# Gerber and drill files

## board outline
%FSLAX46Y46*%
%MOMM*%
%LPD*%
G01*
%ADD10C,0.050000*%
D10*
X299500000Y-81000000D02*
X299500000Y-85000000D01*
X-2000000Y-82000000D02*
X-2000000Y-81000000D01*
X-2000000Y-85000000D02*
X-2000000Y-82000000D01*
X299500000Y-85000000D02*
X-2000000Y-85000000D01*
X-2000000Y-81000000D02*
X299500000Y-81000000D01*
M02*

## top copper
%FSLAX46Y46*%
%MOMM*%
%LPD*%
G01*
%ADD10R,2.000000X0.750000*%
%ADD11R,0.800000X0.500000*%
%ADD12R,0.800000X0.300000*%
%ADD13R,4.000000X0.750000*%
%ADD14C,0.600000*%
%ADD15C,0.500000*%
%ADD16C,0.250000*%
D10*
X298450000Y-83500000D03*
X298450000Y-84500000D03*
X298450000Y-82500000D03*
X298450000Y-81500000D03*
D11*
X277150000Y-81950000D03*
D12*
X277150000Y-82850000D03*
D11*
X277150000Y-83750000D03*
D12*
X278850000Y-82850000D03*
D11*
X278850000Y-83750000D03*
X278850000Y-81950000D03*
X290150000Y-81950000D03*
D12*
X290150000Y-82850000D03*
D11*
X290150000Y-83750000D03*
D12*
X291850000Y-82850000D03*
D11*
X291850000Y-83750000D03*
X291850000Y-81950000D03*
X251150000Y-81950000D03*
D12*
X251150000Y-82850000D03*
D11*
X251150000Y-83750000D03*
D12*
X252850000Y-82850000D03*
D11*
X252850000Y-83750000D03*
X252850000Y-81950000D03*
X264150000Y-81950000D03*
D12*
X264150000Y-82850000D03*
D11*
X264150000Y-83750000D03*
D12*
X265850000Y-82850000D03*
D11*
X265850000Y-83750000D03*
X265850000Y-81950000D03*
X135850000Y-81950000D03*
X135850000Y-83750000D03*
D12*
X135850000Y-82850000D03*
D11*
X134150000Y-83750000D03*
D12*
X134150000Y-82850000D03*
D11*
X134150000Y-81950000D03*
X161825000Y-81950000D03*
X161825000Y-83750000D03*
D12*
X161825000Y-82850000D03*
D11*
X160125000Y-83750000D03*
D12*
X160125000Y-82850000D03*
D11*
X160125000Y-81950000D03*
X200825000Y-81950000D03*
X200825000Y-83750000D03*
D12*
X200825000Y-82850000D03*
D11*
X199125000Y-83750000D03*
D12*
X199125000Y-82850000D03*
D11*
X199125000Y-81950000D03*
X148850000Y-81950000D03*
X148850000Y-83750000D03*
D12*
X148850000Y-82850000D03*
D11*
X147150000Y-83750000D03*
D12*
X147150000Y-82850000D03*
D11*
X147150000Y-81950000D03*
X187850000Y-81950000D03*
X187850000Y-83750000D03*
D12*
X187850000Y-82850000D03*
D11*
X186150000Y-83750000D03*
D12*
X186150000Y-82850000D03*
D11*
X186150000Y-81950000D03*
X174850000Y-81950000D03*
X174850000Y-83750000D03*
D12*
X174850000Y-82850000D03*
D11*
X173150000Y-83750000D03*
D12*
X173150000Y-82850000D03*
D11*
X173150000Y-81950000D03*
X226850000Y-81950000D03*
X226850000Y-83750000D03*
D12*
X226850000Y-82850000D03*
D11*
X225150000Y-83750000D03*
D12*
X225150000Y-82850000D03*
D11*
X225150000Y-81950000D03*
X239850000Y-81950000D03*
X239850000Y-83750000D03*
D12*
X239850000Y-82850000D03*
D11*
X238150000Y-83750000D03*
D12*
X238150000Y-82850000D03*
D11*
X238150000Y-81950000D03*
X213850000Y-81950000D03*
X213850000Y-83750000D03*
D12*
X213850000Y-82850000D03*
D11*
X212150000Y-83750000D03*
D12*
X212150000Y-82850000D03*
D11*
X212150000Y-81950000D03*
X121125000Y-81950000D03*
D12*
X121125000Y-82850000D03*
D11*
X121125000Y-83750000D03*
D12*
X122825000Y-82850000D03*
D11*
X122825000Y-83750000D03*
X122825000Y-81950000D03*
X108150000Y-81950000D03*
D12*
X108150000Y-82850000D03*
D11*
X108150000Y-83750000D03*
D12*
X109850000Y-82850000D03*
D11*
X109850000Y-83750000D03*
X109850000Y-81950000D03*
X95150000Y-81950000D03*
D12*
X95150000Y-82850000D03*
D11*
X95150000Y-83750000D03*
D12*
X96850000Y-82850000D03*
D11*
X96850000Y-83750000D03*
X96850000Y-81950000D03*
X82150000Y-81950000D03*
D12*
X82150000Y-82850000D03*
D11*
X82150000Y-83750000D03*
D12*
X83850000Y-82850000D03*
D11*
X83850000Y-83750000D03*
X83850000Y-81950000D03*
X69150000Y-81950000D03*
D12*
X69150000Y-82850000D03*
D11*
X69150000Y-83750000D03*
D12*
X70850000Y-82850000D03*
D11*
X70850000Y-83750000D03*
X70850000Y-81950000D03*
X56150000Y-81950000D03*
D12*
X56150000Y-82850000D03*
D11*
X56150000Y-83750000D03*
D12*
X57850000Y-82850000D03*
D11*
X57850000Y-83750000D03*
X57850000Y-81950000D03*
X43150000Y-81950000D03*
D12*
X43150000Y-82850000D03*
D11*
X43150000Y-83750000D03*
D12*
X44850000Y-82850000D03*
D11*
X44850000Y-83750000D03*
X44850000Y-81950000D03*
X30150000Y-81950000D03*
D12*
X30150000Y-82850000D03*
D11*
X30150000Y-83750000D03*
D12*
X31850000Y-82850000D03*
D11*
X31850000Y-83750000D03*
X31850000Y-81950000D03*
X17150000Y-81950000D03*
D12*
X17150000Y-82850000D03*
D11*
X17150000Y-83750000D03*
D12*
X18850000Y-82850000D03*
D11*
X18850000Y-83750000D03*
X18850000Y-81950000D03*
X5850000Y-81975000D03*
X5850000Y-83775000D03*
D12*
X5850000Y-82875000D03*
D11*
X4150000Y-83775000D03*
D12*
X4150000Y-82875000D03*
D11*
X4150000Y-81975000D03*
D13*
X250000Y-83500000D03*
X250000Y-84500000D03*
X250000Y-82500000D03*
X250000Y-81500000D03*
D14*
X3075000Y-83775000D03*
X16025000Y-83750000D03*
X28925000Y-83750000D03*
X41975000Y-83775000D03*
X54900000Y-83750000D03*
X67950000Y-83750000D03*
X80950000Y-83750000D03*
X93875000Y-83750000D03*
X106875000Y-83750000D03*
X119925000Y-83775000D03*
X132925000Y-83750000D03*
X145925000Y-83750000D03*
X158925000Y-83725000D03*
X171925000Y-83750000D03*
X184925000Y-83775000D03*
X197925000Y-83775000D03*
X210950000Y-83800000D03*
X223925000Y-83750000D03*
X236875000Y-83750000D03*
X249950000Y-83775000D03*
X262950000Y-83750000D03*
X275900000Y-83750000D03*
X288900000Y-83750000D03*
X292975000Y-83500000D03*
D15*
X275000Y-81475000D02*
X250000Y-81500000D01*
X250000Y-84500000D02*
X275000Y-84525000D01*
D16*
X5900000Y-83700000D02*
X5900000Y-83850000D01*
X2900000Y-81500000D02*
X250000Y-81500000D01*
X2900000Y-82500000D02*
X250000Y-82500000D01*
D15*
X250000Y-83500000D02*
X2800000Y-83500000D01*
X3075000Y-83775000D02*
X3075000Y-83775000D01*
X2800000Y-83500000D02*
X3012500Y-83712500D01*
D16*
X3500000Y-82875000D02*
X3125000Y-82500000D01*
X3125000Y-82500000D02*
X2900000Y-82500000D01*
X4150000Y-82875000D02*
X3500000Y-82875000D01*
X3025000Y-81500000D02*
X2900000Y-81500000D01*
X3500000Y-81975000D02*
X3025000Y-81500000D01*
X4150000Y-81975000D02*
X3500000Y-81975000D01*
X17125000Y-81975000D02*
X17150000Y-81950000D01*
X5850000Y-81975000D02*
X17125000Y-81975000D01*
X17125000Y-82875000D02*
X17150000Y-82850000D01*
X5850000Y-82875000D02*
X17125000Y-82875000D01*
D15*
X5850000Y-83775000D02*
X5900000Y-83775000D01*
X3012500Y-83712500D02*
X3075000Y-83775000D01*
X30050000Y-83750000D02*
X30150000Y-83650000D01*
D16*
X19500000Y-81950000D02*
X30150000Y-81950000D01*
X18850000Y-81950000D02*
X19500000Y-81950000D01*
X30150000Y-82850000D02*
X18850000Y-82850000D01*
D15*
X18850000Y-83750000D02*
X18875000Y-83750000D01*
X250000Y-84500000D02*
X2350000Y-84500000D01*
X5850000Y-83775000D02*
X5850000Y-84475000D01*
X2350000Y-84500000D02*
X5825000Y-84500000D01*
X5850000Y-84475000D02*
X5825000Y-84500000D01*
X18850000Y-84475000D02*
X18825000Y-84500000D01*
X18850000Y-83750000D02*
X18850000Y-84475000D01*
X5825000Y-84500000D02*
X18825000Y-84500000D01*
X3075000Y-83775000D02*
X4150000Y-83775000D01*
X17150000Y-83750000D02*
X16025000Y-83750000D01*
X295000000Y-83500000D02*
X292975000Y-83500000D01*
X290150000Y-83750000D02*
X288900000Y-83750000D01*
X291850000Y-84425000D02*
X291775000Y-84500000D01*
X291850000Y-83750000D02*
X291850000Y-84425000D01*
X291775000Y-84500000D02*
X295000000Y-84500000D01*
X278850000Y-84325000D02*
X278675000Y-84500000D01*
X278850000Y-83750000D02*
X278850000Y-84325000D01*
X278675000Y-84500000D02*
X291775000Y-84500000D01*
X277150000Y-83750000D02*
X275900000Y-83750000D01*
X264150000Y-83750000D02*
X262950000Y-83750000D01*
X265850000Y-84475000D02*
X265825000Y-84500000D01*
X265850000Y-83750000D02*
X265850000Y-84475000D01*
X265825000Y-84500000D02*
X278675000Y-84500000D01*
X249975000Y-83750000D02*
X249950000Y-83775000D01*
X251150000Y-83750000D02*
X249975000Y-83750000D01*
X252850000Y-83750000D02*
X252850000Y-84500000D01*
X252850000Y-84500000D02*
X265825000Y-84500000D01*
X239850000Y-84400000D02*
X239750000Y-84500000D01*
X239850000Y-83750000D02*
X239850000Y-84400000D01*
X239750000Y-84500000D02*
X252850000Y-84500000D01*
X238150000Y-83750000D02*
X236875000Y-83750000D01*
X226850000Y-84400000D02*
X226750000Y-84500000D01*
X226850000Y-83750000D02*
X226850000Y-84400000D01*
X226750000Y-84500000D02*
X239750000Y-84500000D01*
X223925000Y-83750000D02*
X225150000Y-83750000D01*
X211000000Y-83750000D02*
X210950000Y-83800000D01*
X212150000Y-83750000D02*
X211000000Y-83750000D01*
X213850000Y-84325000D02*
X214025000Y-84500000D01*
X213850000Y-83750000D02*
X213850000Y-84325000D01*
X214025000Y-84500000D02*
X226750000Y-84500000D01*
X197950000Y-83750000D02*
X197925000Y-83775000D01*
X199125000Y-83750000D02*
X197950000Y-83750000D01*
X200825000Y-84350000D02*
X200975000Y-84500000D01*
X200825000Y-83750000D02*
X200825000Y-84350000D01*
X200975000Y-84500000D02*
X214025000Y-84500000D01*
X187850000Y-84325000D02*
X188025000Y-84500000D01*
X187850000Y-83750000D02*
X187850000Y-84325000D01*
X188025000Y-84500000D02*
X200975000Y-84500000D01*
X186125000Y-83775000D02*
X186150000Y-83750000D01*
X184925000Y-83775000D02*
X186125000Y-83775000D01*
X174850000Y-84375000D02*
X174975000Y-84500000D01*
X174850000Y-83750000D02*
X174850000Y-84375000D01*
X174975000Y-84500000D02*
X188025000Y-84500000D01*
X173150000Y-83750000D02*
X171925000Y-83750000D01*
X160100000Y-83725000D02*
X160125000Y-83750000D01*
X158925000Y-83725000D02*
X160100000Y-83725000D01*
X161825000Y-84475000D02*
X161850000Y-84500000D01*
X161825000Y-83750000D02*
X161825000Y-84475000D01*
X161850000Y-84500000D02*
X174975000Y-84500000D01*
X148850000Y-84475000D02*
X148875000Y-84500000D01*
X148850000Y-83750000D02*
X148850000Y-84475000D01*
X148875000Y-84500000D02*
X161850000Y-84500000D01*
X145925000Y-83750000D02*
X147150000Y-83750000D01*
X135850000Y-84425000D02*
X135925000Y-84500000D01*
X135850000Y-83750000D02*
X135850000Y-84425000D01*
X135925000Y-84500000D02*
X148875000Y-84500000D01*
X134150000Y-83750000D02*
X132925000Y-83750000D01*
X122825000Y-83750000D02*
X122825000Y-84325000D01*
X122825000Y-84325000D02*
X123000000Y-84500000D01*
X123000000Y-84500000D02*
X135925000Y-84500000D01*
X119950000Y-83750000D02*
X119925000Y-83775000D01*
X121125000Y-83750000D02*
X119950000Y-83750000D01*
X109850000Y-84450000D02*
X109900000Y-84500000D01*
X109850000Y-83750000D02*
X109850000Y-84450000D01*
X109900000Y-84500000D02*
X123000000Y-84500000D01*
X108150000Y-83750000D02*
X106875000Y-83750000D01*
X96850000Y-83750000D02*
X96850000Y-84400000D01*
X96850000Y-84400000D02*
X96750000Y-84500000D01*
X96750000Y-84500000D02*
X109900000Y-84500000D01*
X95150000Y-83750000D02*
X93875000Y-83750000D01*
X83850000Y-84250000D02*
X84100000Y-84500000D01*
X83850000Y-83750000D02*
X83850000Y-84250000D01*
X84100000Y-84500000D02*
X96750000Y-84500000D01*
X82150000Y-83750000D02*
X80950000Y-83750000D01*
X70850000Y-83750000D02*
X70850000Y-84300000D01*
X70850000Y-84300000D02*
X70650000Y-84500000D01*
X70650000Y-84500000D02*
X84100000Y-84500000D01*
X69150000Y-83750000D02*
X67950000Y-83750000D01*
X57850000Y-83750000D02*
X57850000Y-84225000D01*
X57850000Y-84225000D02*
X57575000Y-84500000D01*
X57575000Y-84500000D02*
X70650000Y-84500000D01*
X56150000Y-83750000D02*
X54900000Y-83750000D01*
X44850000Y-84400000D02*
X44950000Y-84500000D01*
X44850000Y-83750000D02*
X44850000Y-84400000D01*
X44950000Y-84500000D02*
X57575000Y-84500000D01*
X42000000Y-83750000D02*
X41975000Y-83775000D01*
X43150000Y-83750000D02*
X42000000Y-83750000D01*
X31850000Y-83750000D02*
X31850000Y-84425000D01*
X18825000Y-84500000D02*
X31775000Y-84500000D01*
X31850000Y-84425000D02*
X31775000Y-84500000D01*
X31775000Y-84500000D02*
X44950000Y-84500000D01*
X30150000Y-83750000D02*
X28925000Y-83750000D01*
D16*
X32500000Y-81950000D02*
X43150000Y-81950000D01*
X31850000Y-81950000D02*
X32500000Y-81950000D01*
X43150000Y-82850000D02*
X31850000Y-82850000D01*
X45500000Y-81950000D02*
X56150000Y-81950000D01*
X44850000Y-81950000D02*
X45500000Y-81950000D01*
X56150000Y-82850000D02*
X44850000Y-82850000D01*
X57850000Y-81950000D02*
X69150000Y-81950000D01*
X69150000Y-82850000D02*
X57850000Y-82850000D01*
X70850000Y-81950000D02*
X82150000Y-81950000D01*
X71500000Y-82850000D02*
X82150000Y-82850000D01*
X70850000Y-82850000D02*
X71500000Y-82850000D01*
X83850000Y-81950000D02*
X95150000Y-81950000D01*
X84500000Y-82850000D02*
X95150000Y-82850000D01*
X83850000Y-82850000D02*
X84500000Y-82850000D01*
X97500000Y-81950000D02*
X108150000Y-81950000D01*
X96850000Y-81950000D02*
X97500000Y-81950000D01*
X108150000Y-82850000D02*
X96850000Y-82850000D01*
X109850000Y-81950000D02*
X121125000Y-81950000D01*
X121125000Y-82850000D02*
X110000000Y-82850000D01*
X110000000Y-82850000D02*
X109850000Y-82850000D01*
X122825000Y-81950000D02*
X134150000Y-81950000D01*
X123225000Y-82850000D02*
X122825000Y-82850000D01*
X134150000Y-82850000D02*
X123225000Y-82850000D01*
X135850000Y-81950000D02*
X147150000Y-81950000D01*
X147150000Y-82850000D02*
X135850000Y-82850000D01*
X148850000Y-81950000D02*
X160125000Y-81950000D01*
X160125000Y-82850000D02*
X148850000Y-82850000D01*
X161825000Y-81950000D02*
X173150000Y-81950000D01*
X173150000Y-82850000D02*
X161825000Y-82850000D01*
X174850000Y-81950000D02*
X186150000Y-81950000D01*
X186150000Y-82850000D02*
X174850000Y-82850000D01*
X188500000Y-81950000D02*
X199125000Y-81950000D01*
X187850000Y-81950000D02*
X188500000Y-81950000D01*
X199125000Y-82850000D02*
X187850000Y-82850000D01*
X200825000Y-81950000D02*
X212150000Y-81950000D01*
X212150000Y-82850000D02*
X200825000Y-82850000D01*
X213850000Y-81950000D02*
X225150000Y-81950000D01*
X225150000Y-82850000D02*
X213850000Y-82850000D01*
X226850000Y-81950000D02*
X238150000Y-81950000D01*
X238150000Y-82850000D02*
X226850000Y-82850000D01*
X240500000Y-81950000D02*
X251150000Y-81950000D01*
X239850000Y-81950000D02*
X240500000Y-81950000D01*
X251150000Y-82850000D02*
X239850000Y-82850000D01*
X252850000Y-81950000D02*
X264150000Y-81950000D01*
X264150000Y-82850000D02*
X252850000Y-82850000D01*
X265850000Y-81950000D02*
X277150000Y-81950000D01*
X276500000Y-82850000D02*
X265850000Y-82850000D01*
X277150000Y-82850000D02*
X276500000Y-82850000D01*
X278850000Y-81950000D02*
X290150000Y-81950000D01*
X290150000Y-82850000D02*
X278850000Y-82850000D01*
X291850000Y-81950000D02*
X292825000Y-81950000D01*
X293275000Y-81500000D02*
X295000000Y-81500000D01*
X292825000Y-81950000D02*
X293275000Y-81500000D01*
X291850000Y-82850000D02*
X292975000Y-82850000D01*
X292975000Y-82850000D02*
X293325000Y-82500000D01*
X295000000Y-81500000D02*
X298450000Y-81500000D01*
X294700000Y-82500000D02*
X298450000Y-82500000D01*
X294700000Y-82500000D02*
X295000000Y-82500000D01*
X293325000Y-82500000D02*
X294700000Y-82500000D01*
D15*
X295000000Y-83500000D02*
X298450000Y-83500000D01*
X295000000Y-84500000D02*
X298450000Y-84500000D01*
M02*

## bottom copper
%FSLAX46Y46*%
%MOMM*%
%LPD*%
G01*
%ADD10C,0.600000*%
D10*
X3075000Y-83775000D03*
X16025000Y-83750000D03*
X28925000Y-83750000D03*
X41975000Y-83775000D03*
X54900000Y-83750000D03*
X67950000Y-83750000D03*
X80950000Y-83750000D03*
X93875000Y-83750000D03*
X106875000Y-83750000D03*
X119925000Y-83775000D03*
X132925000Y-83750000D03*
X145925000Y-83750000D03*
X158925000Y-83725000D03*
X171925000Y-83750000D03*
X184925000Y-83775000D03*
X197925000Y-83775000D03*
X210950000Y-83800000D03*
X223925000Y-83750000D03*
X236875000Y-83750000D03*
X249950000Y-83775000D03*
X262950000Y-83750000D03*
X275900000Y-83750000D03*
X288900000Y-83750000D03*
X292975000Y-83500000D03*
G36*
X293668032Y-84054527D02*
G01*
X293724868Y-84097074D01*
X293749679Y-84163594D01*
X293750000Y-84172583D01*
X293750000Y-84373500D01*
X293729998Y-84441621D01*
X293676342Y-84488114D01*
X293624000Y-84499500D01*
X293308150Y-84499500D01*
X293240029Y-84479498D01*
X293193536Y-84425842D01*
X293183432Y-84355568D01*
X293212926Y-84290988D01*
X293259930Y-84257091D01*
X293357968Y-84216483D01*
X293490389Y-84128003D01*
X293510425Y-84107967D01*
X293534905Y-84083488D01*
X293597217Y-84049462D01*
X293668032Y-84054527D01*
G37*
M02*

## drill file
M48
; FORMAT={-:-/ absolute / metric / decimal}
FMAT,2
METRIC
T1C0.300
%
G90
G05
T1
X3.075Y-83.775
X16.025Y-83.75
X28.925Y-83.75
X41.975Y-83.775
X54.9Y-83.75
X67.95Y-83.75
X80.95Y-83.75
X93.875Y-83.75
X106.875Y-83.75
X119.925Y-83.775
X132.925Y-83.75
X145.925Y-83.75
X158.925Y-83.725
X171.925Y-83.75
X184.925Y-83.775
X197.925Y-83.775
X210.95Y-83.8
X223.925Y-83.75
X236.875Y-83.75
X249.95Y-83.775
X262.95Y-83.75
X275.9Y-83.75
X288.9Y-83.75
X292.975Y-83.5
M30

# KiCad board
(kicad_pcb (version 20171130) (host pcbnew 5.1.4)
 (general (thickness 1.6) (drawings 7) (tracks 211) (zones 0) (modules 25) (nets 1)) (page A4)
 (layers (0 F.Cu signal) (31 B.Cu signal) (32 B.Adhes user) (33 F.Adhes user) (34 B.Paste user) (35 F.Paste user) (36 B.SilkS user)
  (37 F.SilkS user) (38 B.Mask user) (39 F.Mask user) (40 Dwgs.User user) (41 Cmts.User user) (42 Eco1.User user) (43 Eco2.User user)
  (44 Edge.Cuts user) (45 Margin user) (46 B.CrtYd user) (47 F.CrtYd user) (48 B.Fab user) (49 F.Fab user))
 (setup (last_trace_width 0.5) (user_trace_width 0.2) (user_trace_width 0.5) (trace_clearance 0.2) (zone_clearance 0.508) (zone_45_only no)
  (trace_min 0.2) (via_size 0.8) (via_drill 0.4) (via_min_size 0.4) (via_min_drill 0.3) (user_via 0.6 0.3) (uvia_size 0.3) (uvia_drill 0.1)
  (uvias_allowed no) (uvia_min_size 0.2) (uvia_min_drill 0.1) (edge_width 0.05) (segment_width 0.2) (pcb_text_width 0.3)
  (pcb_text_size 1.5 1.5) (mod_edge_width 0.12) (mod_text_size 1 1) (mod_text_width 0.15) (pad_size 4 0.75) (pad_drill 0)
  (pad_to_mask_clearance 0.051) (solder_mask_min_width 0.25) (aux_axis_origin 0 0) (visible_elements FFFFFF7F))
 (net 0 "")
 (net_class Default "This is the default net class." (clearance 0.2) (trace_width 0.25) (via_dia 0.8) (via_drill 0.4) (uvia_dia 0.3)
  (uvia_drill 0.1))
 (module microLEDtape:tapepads (layer F.Cu) (at 281.2 81)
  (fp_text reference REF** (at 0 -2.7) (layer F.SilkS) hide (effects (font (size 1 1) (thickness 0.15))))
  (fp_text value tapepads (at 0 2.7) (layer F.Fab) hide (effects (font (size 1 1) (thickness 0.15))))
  (pad GND smd rect (at 17.25 2.5) (size 2 0.75) (layers F.Cu F.Paste F.Mask))
  (pad VCC smd rect (at 17.25 3.5) (size 2 0.75) (layers F.Cu F.Paste F.Mask))
  (pad CKI smd rect (at 17.25 1.5) (size 2 0.75) (layers F.Cu F.Paste F.Mask))
  (pad SDI smd rect (at 17.25 0.5) (size 2 0.75) (layers F.Cu F.Paste F.Mask)))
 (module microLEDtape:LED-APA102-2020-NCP (layer F.Cu) (at 278 82.85)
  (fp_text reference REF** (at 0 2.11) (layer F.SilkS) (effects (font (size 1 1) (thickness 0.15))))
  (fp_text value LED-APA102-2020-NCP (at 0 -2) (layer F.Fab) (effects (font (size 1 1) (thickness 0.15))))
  (pad SDI smd rect (at -0.85 -0.9) (size 0.8 0.5) (layers F.Cu F.Paste F.Mask))
  (pad CKI smd rect (at -0.85 0) (size 0.8 0.3) (layers F.Cu F.Paste F.Mask))
  (pad GND smd rect (at -0.85 0.9) (size 0.8 0.5) (layers F.Cu F.Paste F.Mask))
  (pad CKO smd rect (at 0.85 0) (size 0.8 0.3) (layers F.Cu F.Paste F.Mask))
  (pad VCC smd rect (at 0.85 0.9) (size 0.8 0.5) (layers F.Cu F.Paste F.Mask))
  (pad SDO smd rect (at 0.85 -0.9) (size 0.8 0.5) (layers F.Cu F.Paste F.Mask)))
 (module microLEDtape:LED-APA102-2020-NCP (layer F.Cu) (at 291 82.85)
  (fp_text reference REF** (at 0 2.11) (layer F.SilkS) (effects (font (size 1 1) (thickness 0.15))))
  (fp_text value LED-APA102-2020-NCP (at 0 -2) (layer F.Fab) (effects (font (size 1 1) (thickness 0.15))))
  (pad SDI smd rect (at -0.85 -0.9) (size 0.8 0.5) (layers F.Cu F.Paste F.Mask))
  (pad CKI smd rect (at -0.85 0) (size 0.8 0.3) (layers F.Cu F.Paste F.Mask))
  (pad GND smd rect (at -0.85 0.9) (size 0.8 0.5) (layers F.Cu F.Paste F.Mask))
  (pad CKO smd rect (at 0.85 0) (size 0.8 0.3) (layers F.Cu F.Paste F.Mask))
  (pad VCC smd rect (at 0.85 0.9) (size 0.8 0.5) (layers F.Cu F.Paste F.Mask))
  (pad SDO smd rect (at 0.85 -0.9) (size 0.8 0.5) (layers F.Cu F.Paste F.Mask)))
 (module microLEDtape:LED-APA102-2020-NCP (layer F.Cu) (at 252 82.85)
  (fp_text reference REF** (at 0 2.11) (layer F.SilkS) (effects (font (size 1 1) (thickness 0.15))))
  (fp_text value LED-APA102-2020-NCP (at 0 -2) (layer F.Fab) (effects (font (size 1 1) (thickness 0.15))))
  (pad SDI smd rect (at -0.85 -0.9) (size 0.8 0.5) (layers F.Cu F.Paste F.Mask))
  (pad CKI smd rect (at -0.85 0) (size 0.8 0.3) (layers F.Cu F.Paste F.Mask))
  (pad GND smd rect (at -0.85 0.9) (size 0.8 0.5) (layers F.Cu F.Paste F.Mask))
  (pad CKO smd rect (at 0.85 0) (size 0.8 0.3) (layers F.Cu F.Paste F.Mask))
  (pad VCC smd rect (at 0.85 0.9) (size 0.8 0.5) (layers F.Cu F.Paste F.Mask))
  (pad SDO smd rect (at 0.85 -0.9) (size 0.8 0.5) (layers F.Cu F.Paste F.Mask)))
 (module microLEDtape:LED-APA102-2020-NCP (layer F.Cu) (at 265 82.85)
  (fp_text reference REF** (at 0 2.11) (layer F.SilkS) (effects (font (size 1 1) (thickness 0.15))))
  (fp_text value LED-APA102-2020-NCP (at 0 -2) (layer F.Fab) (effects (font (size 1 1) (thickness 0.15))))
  (pad SDI smd rect (at -0.85 -0.9) (size 0.8 0.5) (layers F.Cu F.Paste F.Mask))
  (pad CKI smd rect (at -0.85 0) (size 0.8 0.3) (layers F.Cu F.Paste F.Mask))
  (pad GND smd rect (at -0.85 0.9) (size 0.8 0.5) (layers F.Cu F.Paste F.Mask))
  (pad CKO smd rect (at 0.85 0) (size 0.8 0.3) (layers F.Cu F.Paste F.Mask))
  (pad VCC smd rect (at 0.85 0.9) (size 0.8 0.5) (layers F.Cu F.Paste F.Mask))
  (pad SDO smd rect (at 0.85 -0.9) (size 0.8 0.5) (layers F.Cu F.Paste F.Mask)))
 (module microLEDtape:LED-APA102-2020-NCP (layer F.Cu) (at 135 82.85)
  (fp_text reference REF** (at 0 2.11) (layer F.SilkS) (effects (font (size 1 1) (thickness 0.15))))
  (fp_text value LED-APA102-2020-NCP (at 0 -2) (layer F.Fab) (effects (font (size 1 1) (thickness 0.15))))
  (pad SDO smd rect (at 0.85 -0.9) (size 0.8 0.5) (layers F.Cu F.Paste F.Mask))
  (pad VCC smd rect (at 0.85 0.9) (size 0.8 0.5) (layers F.Cu F.Paste F.Mask))
  (pad CKO smd rect (at 0.85 0) (size 0.8 0.3) (layers F.Cu F.Paste F.Mask))
  (pad GND smd rect (at -0.85 0.9) (size 0.8 0.5) (layers F.Cu F.Paste F.Mask))
  (pad CKI smd rect (at -0.85 0) (size 0.8 0.3) (layers F.Cu F.Paste F.Mask))
  (pad SDI smd rect (at -0.85 -0.9) (size 0.8 0.5) (layers F.Cu F.Paste F.Mask)))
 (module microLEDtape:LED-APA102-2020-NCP (layer F.Cu) (at 160.975 82.85)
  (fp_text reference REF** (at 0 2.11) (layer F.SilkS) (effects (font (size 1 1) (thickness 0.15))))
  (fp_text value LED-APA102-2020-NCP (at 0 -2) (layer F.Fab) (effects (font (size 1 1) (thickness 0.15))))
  (pad SDO smd rect (at 0.85 -0.9) (size 0.8 0.5) (layers F.Cu F.Paste F.Mask))
  (pad VCC smd rect (at 0.85 0.9) (size 0.8 0.5) (layers F.Cu F.Paste F.Mask))
  (pad CKO smd rect (at 0.85 0) (size 0.8 0.3) (layers F.Cu F.Paste F.Mask))
  (pad GND smd rect (at -0.85 0.9) (size 0.8 0.5) (layers F.Cu F.Paste F.Mask))
  (pad CKI smd rect (at -0.85 0) (size 0.8 0.3) (layers F.Cu F.Paste F.Mask))
  (pad SDI smd rect (at -0.85 -0.9) (size 0.8 0.5) (layers F.Cu F.Paste F.Mask)))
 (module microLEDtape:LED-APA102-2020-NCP (layer F.Cu) (at 199.975 82.85)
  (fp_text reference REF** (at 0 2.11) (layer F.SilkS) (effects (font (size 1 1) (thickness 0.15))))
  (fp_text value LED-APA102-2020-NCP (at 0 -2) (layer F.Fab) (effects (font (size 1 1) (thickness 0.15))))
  (pad SDO smd rect (at 0.85 -0.9) (size 0.8 0.5) (layers F.Cu F.Paste F.Mask))
  (pad VCC smd rect (at 0.85 0.9) (size 0.8 0.5) (layers F.Cu F.Paste F.Mask))
  (pad CKO smd rect (at 0.85 0) (size 0.8 0.3) (layers F.Cu F.Paste F.Mask))
  (pad GND smd rect (at -0.85 0.9) (size 0.8 0.5) (layers F.Cu F.Paste F.Mask))
  (pad CKI smd rect (at -0.85 0) (size 0.8 0.3) (layers F.Cu F.Paste F.Mask))
  (pad SDI smd rect (at -0.85 -0.9) (size 0.8 0.5) (layers F.Cu F.Paste F.Mask)))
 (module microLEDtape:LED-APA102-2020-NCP (layer F.Cu) (at 148 82.85)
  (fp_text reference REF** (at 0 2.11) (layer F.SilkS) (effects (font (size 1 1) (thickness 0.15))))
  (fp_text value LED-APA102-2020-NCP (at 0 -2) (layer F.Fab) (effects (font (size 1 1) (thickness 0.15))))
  (pad SDO smd rect (at 0.85 -0.9) (size 0.8 0.5) (layers F.Cu F.Paste F.Mask))
  (pad VCC smd rect (at 0.85 0.9) (size 0.8 0.5) (layers F.Cu F.Paste F.Mask))
  (pad CKO smd rect (at 0.85 0) (size 0.8 0.3) (layers F.Cu F.Paste F.Mask))
  (pad GND smd rect (at -0.85 0.9) (size 0.8 0.5) (layers F.Cu F.Paste F.Mask))
  (pad CKI smd rect (at -0.85 0) (size 0.8 0.3) (layers F.Cu F.Paste F.Mask))
  (pad SDI smd rect (at -0.85 -0.9) (size 0.8 0.5) (layers F.Cu F.Paste F.Mask)))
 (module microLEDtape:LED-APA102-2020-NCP (layer F.Cu) (at 187 82.85)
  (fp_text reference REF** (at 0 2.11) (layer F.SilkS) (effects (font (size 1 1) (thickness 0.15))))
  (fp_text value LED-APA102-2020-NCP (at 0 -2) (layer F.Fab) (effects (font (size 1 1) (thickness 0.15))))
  (pad SDO smd rect (at 0.85 -0.9) (size 0.8 0.5) (layers F.Cu F.Paste F.Mask))
  (pad VCC smd rect (at 0.85 0.9) (size 0.8 0.5) (layers F.Cu F.Paste F.Mask))
  (pad CKO smd rect (at 0.85 0) (size 0.8 0.3) (layers F.Cu F.Paste F.Mask))
  (pad GND smd rect (at -0.85 0.9) (size 0.8 0.5) (layers F.Cu F.Paste F.Mask))
  (pad CKI smd rect (at -0.85 0) (size 0.8 0.3) (layers F.Cu F.Paste F.Mask))
  (pad SDI smd rect (at -0.85 -0.9) (size 0.8 0.5) (layers F.Cu F.Paste F.Mask)))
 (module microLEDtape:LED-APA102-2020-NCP (layer F.Cu) (at 174 82.85)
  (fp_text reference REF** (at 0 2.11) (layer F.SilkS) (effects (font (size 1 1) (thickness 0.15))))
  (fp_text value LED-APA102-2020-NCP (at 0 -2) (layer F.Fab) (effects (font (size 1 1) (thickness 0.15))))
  (pad SDO smd rect (at 0.85 -0.9) (size 0.8 0.5) (layers F.Cu F.Paste F.Mask))
  (pad VCC smd rect (at 0.85 0.9) (size 0.8 0.5) (layers F.Cu F.Paste F.Mask))
  (pad CKO smd rect (at 0.85 0) (size 0.8 0.3) (layers F.Cu F.Paste F.Mask))
  (pad GND smd rect (at -0.85 0.9) (size 0.8 0.5) (layers F.Cu F.Paste F.Mask))
  (pad CKI smd rect (at -0.85 0) (size 0.8 0.3) (layers F.Cu F.Paste F.Mask))
  (pad SDI smd rect (at -0.85 -0.9) (size 0.8 0.5) (layers F.Cu F.Paste F.Mask)))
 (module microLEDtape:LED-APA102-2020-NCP (layer F.Cu) (at 226 82.85)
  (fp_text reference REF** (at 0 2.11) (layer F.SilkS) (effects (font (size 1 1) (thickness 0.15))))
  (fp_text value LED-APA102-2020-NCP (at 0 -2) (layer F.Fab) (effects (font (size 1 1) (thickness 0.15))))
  (pad SDO smd rect (at 0.85 -0.9) (size 0.8 0.5) (layers F.Cu F.Paste F.Mask))
  (pad VCC smd rect (at 0.85 0.9) (size 0.8 0.5) (layers F.Cu F.Paste F.Mask))
  (pad CKO smd rect (at 0.85 0) (size 0.8 0.3) (layers F.Cu F.Paste F.Mask))
  (pad GND smd rect (at -0.85 0.9) (size 0.8 0.5) (layers F.Cu F.Paste F.Mask))
  (pad CKI smd rect (at -0.85 0) (size 0.8 0.3) (layers F.Cu F.Paste F.Mask))
  (pad SDI smd rect (at -0.85 -0.9) (size 0.8 0.5) (layers F.Cu F.Paste F.Mask)))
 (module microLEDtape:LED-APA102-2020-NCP (layer F.Cu) (at 239 82.85)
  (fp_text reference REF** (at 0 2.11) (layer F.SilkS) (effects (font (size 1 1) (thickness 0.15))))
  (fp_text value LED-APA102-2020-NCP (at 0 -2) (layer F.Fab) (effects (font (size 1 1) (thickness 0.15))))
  (pad SDO smd rect (at 0.85 -0.9) (size 0.8 0.5) (layers F.Cu F.Paste F.Mask))
  (pad VCC smd rect (at 0.85 0.9) (size 0.8 0.5) (layers F.Cu F.Paste F.Mask))
  (pad CKO smd rect (at 0.85 0) (size 0.8 0.3) (layers F.Cu F.Paste F.Mask))
  (pad GND smd rect (at -0.85 0.9) (size 0.8 0.5) (layers F.Cu F.Paste F.Mask))
  (pad CKI smd rect (at -0.85 0) (size 0.8 0.3) (layers F.Cu F.Paste F.Mask))
  (pad SDI smd rect (at -0.85 -0.9) (size 0.8 0.5) (layers F.Cu F.Paste F.Mask)))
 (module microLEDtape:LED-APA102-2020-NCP (layer F.Cu) (at 213 82.85)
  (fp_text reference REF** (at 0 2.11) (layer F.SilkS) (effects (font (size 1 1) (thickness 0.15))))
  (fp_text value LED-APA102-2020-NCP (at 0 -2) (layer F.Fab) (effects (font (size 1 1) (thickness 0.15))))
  (pad SDO smd rect (at 0.85 -0.9) (size 0.8 0.5) (layers F.Cu F.Paste F.Mask))
  (pad VCC smd rect (at 0.85 0.9) (size 0.8 0.5) (layers F.Cu F.Paste F.Mask))
  (pad CKO smd rect (at 0.85 0) (size 0.8 0.3) (layers F.Cu F.Paste F.Mask))
  (pad GND smd rect (at -0.85 0.9) (size 0.8 0.5) (layers F.Cu F.Paste F.Mask))
  (pad CKI smd rect (at -0.85 0) (size 0.8 0.3) (layers F.Cu F.Paste F.Mask))
  (pad SDI smd rect (at -0.85 -0.9) (size 0.8 0.5) (layers F.Cu F.Paste F.Mask)))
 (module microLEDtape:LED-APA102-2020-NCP (layer F.Cu) (at 121.975 82.85)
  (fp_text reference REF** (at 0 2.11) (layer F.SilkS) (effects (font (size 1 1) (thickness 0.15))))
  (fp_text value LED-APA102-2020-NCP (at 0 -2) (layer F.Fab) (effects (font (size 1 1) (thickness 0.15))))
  (pad SDI smd rect (at -0.85 -0.9) (size 0.8 0.5) (layers F.Cu F.Paste F.Mask))
  (pad CKI smd rect (at -0.85 0) (size 0.8 0.3) (layers F.Cu F.Paste F.Mask))
  (pad GND smd rect (at -0.85 0.9) (size 0.8 0.5) (layers F.Cu F.Paste F.Mask))
  (pad CKO smd rect (at 0.85 0) (size 0.8 0.3) (layers F.Cu F.Paste F.Mask))
  (pad VCC smd rect (at 0.85 0.9) (size 0.8 0.5) (layers F.Cu F.Paste F.Mask))
  (pad SDO smd rect (at 0.85 -0.9) (size 0.8 0.5) (layers F.Cu F.Paste F.Mask)))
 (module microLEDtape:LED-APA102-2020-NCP (layer F.Cu) (at 109 82.85)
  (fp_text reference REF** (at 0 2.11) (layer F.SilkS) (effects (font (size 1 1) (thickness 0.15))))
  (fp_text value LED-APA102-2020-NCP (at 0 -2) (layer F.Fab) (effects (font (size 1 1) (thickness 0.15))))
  (pad SDI smd rect (at -0.85 -0.9) (size 0.8 0.5) (layers F.Cu F.Paste F.Mask))
  (pad CKI smd rect (at -0.85 0) (size 0.8 0.3) (layers F.Cu F.Paste F.Mask))
  (pad GND smd rect (at -0.85 0.9) (size 0.8 0.5) (layers F.Cu F.Paste F.Mask))
  (pad CKO smd rect (at 0.85 0) (size 0.8 0.3) (layers F.Cu F.Paste F.Mask))
  (pad VCC smd rect (at 0.85 0.9) (size 0.8 0.5) (layers F.Cu F.Paste F.Mask))
  (pad SDO smd rect (at 0.85 -0.9) (size 0.8 0.5) (layers F.Cu F.Paste F.Mask)))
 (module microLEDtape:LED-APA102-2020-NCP (layer F.Cu) (at 96 82.85)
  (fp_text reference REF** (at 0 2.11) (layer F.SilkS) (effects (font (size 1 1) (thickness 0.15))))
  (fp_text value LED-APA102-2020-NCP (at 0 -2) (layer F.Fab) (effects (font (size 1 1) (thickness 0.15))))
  (pad SDI smd rect (at -0.85 -0.9) (size 0.8 0.5) (layers F.Cu F.Paste F.Mask))
  (pad CKI smd rect (at -0.85 0) (size 0.8 0.3) (layers F.Cu F.Paste F.Mask))
  (pad GND smd rect (at -0.85 0.9) (size 0.8 0.5) (layers F.Cu F.Paste F.Mask))
  (pad CKO smd rect (at 0.85 0) (size 0.8 0.3) (layers F.Cu F.Paste F.Mask))
  (pad VCC smd rect (at 0.85 0.9) (size 0.8 0.5) (layers F.Cu F.Paste F.Mask))
  (pad SDO smd rect (at 0.85 -0.9) (size 0.8 0.5) (layers F.Cu F.Paste F.Mask)))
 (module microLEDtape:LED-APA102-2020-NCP (layer F.Cu) (at 83 82.85)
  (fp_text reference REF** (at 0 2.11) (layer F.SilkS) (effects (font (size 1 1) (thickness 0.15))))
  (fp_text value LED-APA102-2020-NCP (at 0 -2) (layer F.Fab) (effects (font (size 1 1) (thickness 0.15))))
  (pad SDI smd rect (at -0.85 -0.9) (size 0.8 0.5) (layers F.Cu F.Paste F.Mask))
  (pad CKI smd rect (at -0.85 0) (size 0.8 0.3) (layers F.Cu F.Paste F.Mask))
  (pad GND smd rect (at -0.85 0.9) (size 0.8 0.5) (layers F.Cu F.Paste F.Mask))
  (pad CKO smd rect (at 0.85 0) (size 0.8 0.3) (layers F.Cu F.Paste F.Mask))
  (pad VCC smd rect (at 0.85 0.9) (size 0.8 0.5) (layers F.Cu F.Paste F.Mask))
  (pad SDO smd rect (at 0.85 -0.9) (size 0.8 0.5) (layers F.Cu F.Paste F.Mask)))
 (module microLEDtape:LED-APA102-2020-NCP (layer F.Cu) (at 70 82.85)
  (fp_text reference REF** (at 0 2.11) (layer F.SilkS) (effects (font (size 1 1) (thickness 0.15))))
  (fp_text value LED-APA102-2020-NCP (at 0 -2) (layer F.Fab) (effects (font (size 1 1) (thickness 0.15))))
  (pad SDI smd rect (at -0.85 -0.9) (size 0.8 0.5) (layers F.Cu F.Paste F.Mask))
  (pad CKI smd rect (at -0.85 0) (size 0.8 0.3) (layers F.Cu F.Paste F.Mask))
  (pad GND smd rect (at -0.85 0.9) (size 0.8 0.5) (layers F.Cu F.Paste F.Mask))
  (pad CKO smd rect (at 0.85 0) (size 0.8 0.3) (layers F.Cu F.Paste F.Mask))
  (pad VCC smd rect (at 0.85 0.9) (size 0.8 0.5) (layers F.Cu F.Paste F.Mask))
  (pad SDO smd rect (at 0.85 -0.9) (size 0.8 0.5) (layers F.Cu F.Paste F.Mask)))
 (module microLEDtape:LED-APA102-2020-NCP (layer F.Cu) (at 57 82.85)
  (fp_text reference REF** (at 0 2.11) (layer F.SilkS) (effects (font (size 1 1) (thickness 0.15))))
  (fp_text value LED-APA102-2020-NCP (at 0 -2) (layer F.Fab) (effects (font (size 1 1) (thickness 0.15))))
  (pad SDI smd rect (at -0.85 -0.9) (size 0.8 0.5) (layers F.Cu F.Paste F.Mask))
  (pad CKI smd rect (at -0.85 0) (size 0.8 0.3) (layers F.Cu F.Paste F.Mask))
  (pad GND smd rect (at -0.85 0.9) (size 0.8 0.5) (layers F.Cu F.Paste F.Mask))
  (pad CKO smd rect (at 0.85 0) (size 0.8 0.3) (layers F.Cu F.Paste F.Mask))
  (pad VCC smd rect (at 0.85 0.9) (size 0.8 0.5) (layers F.Cu F.Paste F.Mask))
  (pad SDO smd rect (at 0.85 -0.9) (size 0.8 0.5) (layers F.Cu F.Paste F.Mask)))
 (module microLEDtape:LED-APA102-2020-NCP (layer F.Cu) (at 44 82.85)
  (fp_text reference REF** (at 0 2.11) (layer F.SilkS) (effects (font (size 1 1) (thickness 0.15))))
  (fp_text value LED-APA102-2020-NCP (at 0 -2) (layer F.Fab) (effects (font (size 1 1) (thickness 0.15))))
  (pad SDI smd rect (at -0.85 -0.9) (size 0.8 0.5) (layers F.Cu F.Paste F.Mask))
  (pad CKI smd rect (at -0.85 0) (size 0.8 0.3) (layers F.Cu F.Paste F.Mask))
  (pad GND smd rect (at -0.85 0.9) (size 0.8 0.5) (layers F.Cu F.Paste F.Mask))
  (pad CKO smd rect (at 0.85 0) (size 0.8 0.3) (layers F.Cu F.Paste F.Mask))
  (pad VCC smd rect (at 0.85 0.9) (size 0.8 0.5) (layers F.Cu F.Paste F.Mask))
  (pad SDO smd rect (at 0.85 -0.9) (size 0.8 0.5) (layers F.Cu F.Paste F.Mask)))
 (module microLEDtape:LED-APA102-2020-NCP (layer F.Cu) (at 31 82.85)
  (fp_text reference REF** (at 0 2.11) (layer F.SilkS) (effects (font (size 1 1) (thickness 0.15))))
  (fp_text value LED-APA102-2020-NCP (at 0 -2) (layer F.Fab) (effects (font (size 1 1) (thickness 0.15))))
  (pad SDI smd rect (at -0.85 -0.9) (size 0.8 0.5) (layers F.Cu F.Paste F.Mask))
  (pad CKI smd rect (at -0.85 0) (size 0.8 0.3) (layers F.Cu F.Paste F.Mask))
  (pad GND smd rect (at -0.85 0.9) (size 0.8 0.5) (layers F.Cu F.Paste F.Mask))
  (pad CKO smd rect (at 0.85 0) (size 0.8 0.3) (layers F.Cu F.Paste F.Mask))
  (pad VCC smd rect (at 0.85 0.9) (size 0.8 0.5) (layers F.Cu F.Paste F.Mask))
  (pad SDO smd rect (at 0.85 -0.9) (size 0.8 0.5) (layers F.Cu F.Paste F.Mask)))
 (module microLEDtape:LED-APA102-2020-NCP (layer F.Cu) (at 18 82.85)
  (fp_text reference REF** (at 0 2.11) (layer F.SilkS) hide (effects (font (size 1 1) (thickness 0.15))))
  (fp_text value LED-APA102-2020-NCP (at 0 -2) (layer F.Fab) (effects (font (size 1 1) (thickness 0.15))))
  (pad SDI smd rect (at -0.85 -0.9) (size 0.8 0.5) (layers F.Cu F.Paste F.Mask))
  (pad CKI smd rect (at -0.85 0) (size 0.8 0.3) (layers F.Cu F.Paste F.Mask))
  (pad GND smd rect (at -0.85 0.9) (size 0.8 0.5) (layers F.Cu F.Paste F.Mask))
  (pad CKO smd rect (at 0.85 0) (size 0.8 0.3) (layers F.Cu F.Paste F.Mask))
  (pad VCC smd rect (at 0.85 0.9) (size 0.8 0.5) (layers F.Cu F.Paste F.Mask))
  (pad SDO smd rect (at 0.85 -0.9) (size 0.8 0.5) (layers F.Cu F.Paste F.Mask)))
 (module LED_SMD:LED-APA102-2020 (layer F.Cu) (at 5 82.875)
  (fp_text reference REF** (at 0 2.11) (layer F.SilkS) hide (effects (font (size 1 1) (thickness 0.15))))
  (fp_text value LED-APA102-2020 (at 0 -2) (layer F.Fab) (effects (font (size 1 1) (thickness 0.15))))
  (pad SDO smd rect (at 0.85 -0.9) (size 0.8 0.5) (layers F.Cu F.Paste F.Mask))
  (pad VCC smd rect (at 0.85 0.9) (size 0.8 0.5) (layers F.Cu F.Paste F.Mask))
  (pad CKO smd rect (at 0.85 0) (size 0.8 0.3) (layers F.Cu F.Paste F.Mask))
  (pad GND smd rect (at -0.85 0.9) (size 0.8 0.5) (layers F.Cu F.Paste F.Mask))
  (pad CKI smd rect (at -0.85 0) (size 0.8 0.3) (layers F.Cu F.Paste F.Mask))
  (pad SDI smd rect (at -0.85 -0.9) (size 0.8 0.5) (layers F.Cu F.Paste F.Mask)))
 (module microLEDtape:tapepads (layer F.Cu) (at -17 81)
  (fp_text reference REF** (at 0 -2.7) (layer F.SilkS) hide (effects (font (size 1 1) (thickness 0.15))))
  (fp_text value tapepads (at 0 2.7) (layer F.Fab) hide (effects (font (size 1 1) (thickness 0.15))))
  (pad GND smd rect (at 17.25 2.5) (size 4 0.75) (layers F.Cu F.Paste F.Mask))
  (pad VCC smd rect (at 17.25 3.5) (size 4 0.75) (layers F.Cu F.Paste F.Mask))
  (pad CKI smd rect (at 17.25 1.5) (size 4 0.75) (layers F.Cu F.Paste F.Mask))
  (pad SDI smd rect (at 17.25 0.5) (size 4 0.75) (layers F.Cu F.Paste F.Mask)))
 (gr_line (start 299.5 81) (end 299.5 85) (layer Edge.Cuts) (width 0.05))
 (gr_line (start -2 82) (end -2 81) (layer Edge.Cuts) (width 0.05))
 (gr_line (start -2 85) (end -2 82) (layer Edge.Cuts) (width 0.05))
 (gr_line (start 299.5 85) (end -2 85) (layer Edge.Cuts) (width 0.05))
 (gr_line (start -2 81) (end 299.5 81) (layer Edge.Cuts) (width 0.05))
 (segment (start 0.275 81.475) (end 0.25 81.5) (width 0.5) (layer F.Cu) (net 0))
 (segment (start 0.25 84.5) (end 0.275 84.525) (width 0.5) (layer F.Cu) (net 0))
 (segment (start 5.9 83.7) (end 5.9 83.85) (width 0.25) (layer F.Cu) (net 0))
 (segment (start 2.9 81.5) (end 0.25 81.5) (width 0.25) (layer F.Cu) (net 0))
 (segment (start 2.9 82.5) (end 0.25 82.5) (width 0.25) (layer F.Cu) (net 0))
 (segment (start 0.25 83.5) (end 2.8 83.5) (width 0.5) (layer F.Cu) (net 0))
 (segment (start 3.075 83.775) (end 3.075 83.775) (width 0.5) (layer F.Cu) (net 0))
 (segment (start 2.8 83.5) (end 3.0125 83.7125) (width 0.5) (layer F.Cu) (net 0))
 (segment (start 3.5 82.875) (end 3.125 82.5) (width 0.25) (layer F.Cu) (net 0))
 (segment (start 3.125 82.5) (end 2.9 82.5) (width 0.25) (layer F.Cu) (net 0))
 (segment (start 4.15 82.875) (end 3.5 82.875) (width 0.25) (layer F.Cu) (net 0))
 (segment (start 3.025 81.5) (end 2.9 81.5) (width 0.25) (layer F.Cu) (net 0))
 (segment (start 3.5 81.975) (end 3.025 81.5) (width 0.25) (layer F.Cu) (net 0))
 (segment (start 4.15 81.975) (end 3.5 81.975) (width 0.25) (layer F.Cu) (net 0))
 (segment (start 17.125 81.975) (end 17.15 81.95) (width 0.25) (layer F.Cu) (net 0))
 (segment (start 5.85 81.975) (end 17.125 81.975) (width 0.25) (layer F.Cu) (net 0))
 (segment (start 17.125 82.875) (end 17.15 82.85) (width 0.25) (layer F.Cu) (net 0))
 (segment (start 5.85 82.875) (end 17.125 82.875) (width 0.25) (layer F.Cu) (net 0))
 (segment (start 5.85 83.775) (end 5.9 83.775) (width 0.5) (layer F.Cu) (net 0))
 (segment (start 3.0125 83.7125) (end 3.075 83.775) (width 0.5) (layer F.Cu) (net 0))
 (segment (start 30.05 83.75) (end 30.15 83.65) (width 0.5) (layer F.Cu) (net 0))
 (segment (start 19.5 81.95) (end 30.15 81.95) (width 0.25) (layer F.Cu) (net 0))
 (segment (start 18.85 81.95) (end 19.5 81.95) (width 0.25) (layer F.Cu) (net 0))
 (segment (start 30.15 82.85) (end 18.85 82.85) (width 0.25) (layer F.Cu) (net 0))
 (segment (start 18.85 83.75) (end 18.875 83.75) (width 0.5) (layer F.Cu) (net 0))
 (segment (start 0.25 84.5) (end 2.35 84.5) (width 0.5) (layer F.Cu) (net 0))
 (segment (start 5.85 83.775) (end 5.85 84.475) (width 0.5) (layer F.Cu) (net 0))
 (segment (start 2.35 84.5) (end 5.825 84.5) (width 0.5) (layer F.Cu) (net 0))
 (segment (start 5.85 84.475) (end 5.825 84.5) (width 0.5) (layer F.Cu) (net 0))
 (segment (start 18.85 84.475) (end 18.825 84.5) (width 0.5) (layer F.Cu) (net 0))
 (segment (start 18.85 83.75) (end 18.85 84.475) (width 0.5) (layer F.Cu) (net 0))
 (segment (start 5.825 84.5) (end 18.825 84.5) (width 0.5) (layer F.Cu) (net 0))
 (segment (start 3.075 83.775) (end 4.15 83.775) (width 0.5) (layer F.Cu) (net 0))
 (via (at 3.075 83.775) (size 0.6) (drill 0.3) (layers F.Cu B.Cu) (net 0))
 (via (at 16.025 83.75) (size 0.6) (drill 0.3) (layers F.Cu B.Cu) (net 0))
 (segment (start 17.15 83.75) (end 16.025 83.75) (width 0.5) (layer F.Cu) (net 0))
 (via (at 28.925 83.75) (size 0.6) (drill 0.3) (layers F.Cu B.Cu) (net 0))
 (via (at 41.975 83.775) (size 0.6) (drill 0.3) (layers F.Cu B.Cu) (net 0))
 (via (at 54.9 83.75) (size 0.6) (drill 0.3) (layers F.Cu B.Cu) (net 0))
 (via (at 67.95 83.75) (size 0.6) (drill 0.3) (layers F.Cu B.Cu) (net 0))
 (via (at 80.95 83.75) (size 0.6) (drill 0.3) (layers F.Cu B.Cu) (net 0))
 (via (at 93.875 83.75) (size 0.6) (drill 0.3) (layers F.Cu B.Cu) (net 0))
 (via (at 106.875 83.75) (size 0.6) (drill 0.3) (layers F.Cu B.Cu) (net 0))
 (via (at 119.925 83.775) (size 0.6) (drill 0.3) (layers F.Cu B.Cu) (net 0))
 (via (at 132.925 83.75) (size 0.6) (drill 0.3) (layers F.Cu B.Cu) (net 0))
 (via (at 145.925 83.75) (size 0.6) (drill 0.3) (layers F.Cu B.Cu) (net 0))
 (via (at 158.925 83.725) (size 0.6) (drill 0.3) (layers F.Cu B.Cu) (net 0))
 (via (at 171.925 83.75) (size 0.6) (drill 0.3) (layers F.Cu B.Cu) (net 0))
 (via (at 184.925 83.775) (size 0.6) (drill 0.3) (layers F.Cu B.Cu) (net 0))
 (via (at 197.925 83.775) (size 0.6) (drill 0.3) (layers F.Cu B.Cu) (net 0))
 (via (at 210.95 83.8) (size 0.6) (drill 0.3) (layers F.Cu B.Cu) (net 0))
 (via (at 223.925 83.75) (size 0.6) (drill 0.3) (layers F.Cu B.Cu) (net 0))
 (via (at 236.875 83.75) (size 0.6) (drill 0.3) (layers F.Cu B.Cu) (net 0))
 (via (at 249.95 83.775) (size 0.6) (drill 0.3) (layers F.Cu B.Cu) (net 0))
 (via (at 262.95 83.75) (size 0.6) (drill 0.3) (layers F.Cu B.Cu) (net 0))
 (via (at 275.9 83.75) (size 0.6) (drill 0.3) (layers F.Cu B.Cu) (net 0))
 (via (at 288.9 83.75) (size 0.6) (drill 0.3) (layers F.Cu B.Cu) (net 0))
 (via (at 292.975 83.5) (size 0.6) (drill 0.3) (layers F.Cu B.Cu) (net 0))
 (segment (start 295 83.5) (end 292.975 83.5) (width 0.5) (layer F.Cu) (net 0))
 (segment (start 290.15 83.75) (end 288.9 83.75) (width 0.5) (layer F.Cu) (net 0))
 (segment (start 291.85 84.425) (end 291.775 84.5) (width 0.5) (layer F.Cu) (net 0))
 (segment (start 291.85 83.75) (end 291.85 84.425) (width 0.5) (layer F.Cu) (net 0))
 (segment (start 291.775 84.5) (end 295 84.5) (width 0.5) (layer F.Cu) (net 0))
 (segment (start 278.85 84.325) (end 278.675 84.5) (width 0.5) (layer F.Cu) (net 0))
 (segment (start 278.85 83.75) (end 278.85 84.325) (width 0.5) (layer F.Cu) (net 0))
 (segment (start 278.675 84.5) (end 291.775 84.5) (width 0.5) (layer F.Cu) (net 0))
 (segment (start 277.15 83.75) (end 275.9 83.75) (width 0.5) (layer F.Cu) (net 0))
 (segment (start 264.15 83.75) (end 262.95 83.75) (width 0.5) (layer F.Cu) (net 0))
 (segment (start 265.85 84.475) (end 265.825 84.5) (width 0.5) (layer F.Cu) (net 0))
 (segment (start 265.85 83.75) (end 265.85 84.475) (width 0.5) (layer F.Cu) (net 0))
 (segment (start 265.825 84.5) (end 278.675 84.5) (width 0.5) (layer F.Cu) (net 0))
 (segment (start 249.975 83.75) (end 249.95 83.775) (width 0.5) (layer F.Cu) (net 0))
 (segment (start 251.15 83.75) (end 249.975 83.75) (width 0.5) (layer F.Cu) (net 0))
 (segment (start 252.85 83.75) (end 252.85 84.5) (width 0.5) (layer F.Cu) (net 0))
 (segment (start 252.85 84.5) (end 265.825 84.5) (width 0.5) (layer F.Cu) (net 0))
 (segment (start 239.85 84.4) (end 239.75 84.5) (width 0.5) (layer F.Cu) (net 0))
 (segment (start 239.85 83.75) (end 239.85 84.4) (width 0.5) (layer F.Cu) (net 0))
 (segment (start 239.75 84.5) (end 252.85 84.5) (width 0.5) (layer F.Cu) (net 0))
 (segment (start 238.15 83.75) (end 236.875 83.75) (width 0.5) (layer F.Cu) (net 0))
 (segment (start 226.85 84.4) (end 226.75 84.5) (width 0.5) (layer F.Cu) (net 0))
 (segment (start 226.85 83.75) (end 226.85 84.4) (width 0.5) (layer F.Cu) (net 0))
 (segment (start 226.75 84.5) (end 239.75 84.5) (width 0.5) (layer F.Cu) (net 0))
 (segment (start 223.925 83.75) (end 225.15 83.75) (width 0.5) (layer F.Cu) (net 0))
 (segment (start 211 83.75) (end 210.95 83.8) (width 0.5) (layer F.Cu) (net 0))
 (segment (start 212.15 83.75) (end 211 83.75) (width 0.5) (layer F.Cu) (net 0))
 (segment (start 213.85 84.325) (end 214.025 84.5) (width 0.5) (layer F.Cu) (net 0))
 (segment (start 213.85 83.75) (end 213.85 84.325) (width 0.5) (layer F.Cu) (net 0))
 (segment (start 214.025 84.5) (end 226.75 84.5) (width 0.5) (layer F.Cu) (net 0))
 (segment (start 197.95 83.75) (end 197.925 83.775) (width 0.5) (layer F.Cu) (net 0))
 (segment (start 199.125 83.75) (end 197.95 83.75) (width 0.5) (layer F.Cu) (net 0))
 (segment (start 200.825 84.35) (end 200.975 84.5) (width 0.5) (layer F.Cu) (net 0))
 (segment (start 200.825 83.75) (end 200.825 84.35) (width 0.5) (layer F.Cu) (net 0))
 (segment (start 200.975 84.5) (end 214.025 84.5) (width 0.5) (layer F.Cu) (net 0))
 (segment (start 187.85 84.325) (end 188.025 84.5) (width 0.5) (layer F.Cu) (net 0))
 (segment (start 187.85 83.75) (end 187.85 84.325) (width 0.5) (layer F.Cu) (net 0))
 (segment (start 188.025 84.5) (end 200.975 84.5) (width 0.5) (layer F.Cu) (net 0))
 (segment (start 186.125 83.775) (end 186.15 83.75) (width 0.5) (layer F.Cu) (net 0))
 (segment (start 184.925 83.775) (end 186.125 83.775) (width 0.5) (layer F.Cu) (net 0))
 (segment (start 174.85 84.375) (end 174.975 84.5) (width 0.5) (layer F.Cu) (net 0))
 (segment (start 174.85 83.75) (end 174.85 84.375) (width 0.5) (layer F.Cu) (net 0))
 (segment (start 174.975 84.5) (end 188.025 84.5) (width 0.5) (layer F.Cu) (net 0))
 (segment (start 173.15 83.75) (end 171.925 83.75) (width 0.5) (layer F.Cu) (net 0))
 (segment (start 160.1 83.725) (end 160.125 83.75) (width 0.5) (layer F.Cu) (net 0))
 (segment (start 158.925 83.725) (end 160.1 83.725) (width 0.5) (layer F.Cu) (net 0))
 (segment (start 161.825 84.475) (end 161.85 84.5) (width 0.5) (layer F.Cu) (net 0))
 (segment (start 161.825 83.75) (end 161.825 84.475) (width 0.5) (layer F.Cu) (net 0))
 (segment (start 161.85 84.5) (end 174.975 84.5) (width 0.5) (layer F.Cu) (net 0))
 (segment (start 148.85 84.475) (end 148.875 84.5) (width 0.5) (layer F.Cu) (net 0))
 (segment (start 148.85 83.75) (end 148.85 84.475) (width 0.5) (layer F.Cu) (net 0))
 (segment (start 148.875 84.5) (end 161.85 84.5) (width 0.5) (layer F.Cu) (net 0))
 (segment (start 145.925 83.75) (end 147.15 83.75) (width 0.5) (layer F.Cu) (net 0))
 (segment (start 135.85 84.425) (end 135.925 84.5) (width 0.5) (layer F.Cu) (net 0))
 (segment (start 135.85 83.75) (end 135.85 84.425) (width 0.5) (layer F.Cu) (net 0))
 (segment (start 135.925 84.5) (end 148.875 84.5) (width 0.5) (layer F.Cu) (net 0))
 (segment (start 134.15 83.75) (end 132.925 83.75) (width 0.5) (layer F.Cu) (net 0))
 (segment (start 122.825 83.75) (end 122.825 84.325) (width 0.5) (layer F.Cu) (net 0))
 (segment (start 122.825 84.325) (end 123 84.5) (width 0.5) (layer F.Cu) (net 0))
 (segment (start 123 84.5) (end 135.925 84.5) (width 0.5) (layer F.Cu) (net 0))
 (segment (start 119.95 83.75) (end 119.925 83.775) (width 0.5) (layer F.Cu) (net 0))
 (segment (start 121.125 83.75) (end 119.95 83.75) (width 0.5) (layer F.Cu) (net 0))
 (segment (start 109.85 84.45) (end 109.9 84.5) (width 0.5) (layer F.Cu) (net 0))
 (segment (start 109.85 83.75) (end 109.85 84.45) (width 0.5) (layer F.Cu) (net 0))
 (segment (start 109.9 84.5) (end 123 84.5) (width 0.5) (layer F.Cu) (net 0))
 (segment (start 108.15 83.75) (end 106.875 83.75) (width 0.5) (layer F.Cu) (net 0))
 (segment (start 96.85 83.75) (end 96.85 84.4) (width 0.5) (layer F.Cu) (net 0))
 (segment (start 96.85 84.4) (end 96.75 84.5) (width 0.5) (layer F.Cu) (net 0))
 (segment (start 96.75 84.5) (end 109.9 84.5) (width 0.5) (layer F.Cu) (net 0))
 (segment (start 95.15 83.75) (end 93.875 83.75) (width 0.5) (layer F.Cu) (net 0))
 (segment (start 83.85 84.25) (end 84.1 84.5) (width 0.5) (layer F.Cu) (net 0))
 (segment (start 83.85 83.75) (end 83.85 84.25) (width 0.5) (layer F.Cu) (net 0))
 (segment (start 84.1 84.5) (end 96.75 84.5) (width 0.5) (layer F.Cu) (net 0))
 (segment (start 82.15 83.75) (end 80.95 83.75) (width 0.5) (layer F.Cu) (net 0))
 (segment (start 70.85 83.75) (end 70.85 84.3) (width 0.5) (layer F.Cu) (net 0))
 (segment (start 70.85 84.3) (end 70.65 84.5) (width 0.5) (layer F.Cu) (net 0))
 (segment (start 70.65 84.5) (end 84.1 84.5) (width 0.5) (layer F.Cu) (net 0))
 (segment (start 69.15 83.75) (end 67.95 83.75) (width 0.5) (layer F.Cu) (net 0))
 (segment (start 57.85 83.75) (end 57.85 84.225) (width 0.5) (layer F.Cu) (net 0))
 (segment (start 57.85 84.225) (end 57.575 84.5) (width 0.5) (layer F.Cu) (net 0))
 (segment (start 57.575 84.5) (end 70.65 84.5) (width 0.5) (layer F.Cu) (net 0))
 (segment (start 56.15 83.75) (end 54.9 83.75) (width 0.5) (layer F.Cu) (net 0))
 (segment (start 44.85 84.4) (end 44.95 84.5) (width 0.5) (layer F.Cu) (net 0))
 (segment (start 44.85 83.75) (end 44.85 84.4) (width 0.5) (layer F.Cu) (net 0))
 (segment (start 44.95 84.5) (end 57.575 84.5) (width 0.5) (layer F.Cu) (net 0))
 (segment (start 42 83.75) (end 41.975 83.775) (width 0.5) (layer F.Cu) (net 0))
 (segment (start 43.15 83.75) (end 42 83.75) (width 0.5) (layer F.Cu) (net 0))
 (segment (start 31.85 83.75) (end 31.85 84.425) (width 0.5) (layer F.Cu) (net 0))
 (segment (start 18.825 84.5) (end 31.775 84.5) (width 0.5) (layer F.Cu) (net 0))
 (segment (start 31.85 84.425) (end 31.775 84.5) (width 0.5) (layer F.Cu) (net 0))
 (segment (start 31.775 84.5) (end 44.95 84.5) (width 0.5) (layer F.Cu) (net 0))
 (segment (start 30.15 83.75) (end 28.925 83.75) (width 0.5) (layer F.Cu) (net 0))
 (segment (start 32.5 81.95) (end 43.15 81.95) (width 0.25) (layer F.Cu) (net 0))
 (segment (start 31.85 81.95) (end 32.5 81.95) (width 0.25) (layer F.Cu) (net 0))
 (segment (start 43.15 82.85) (end 31.85 82.85) (width 0.25) (layer F.Cu) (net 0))
 (segment (start 45.5 81.95) (end 56.15 81.95) (width 0.25) (layer F.Cu) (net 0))
 (segment (start 44.85 81.95) (end 45.5 81.95) (width 0.25) (layer F.Cu) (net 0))
 (segment (start 56.15 82.85) (end 44.85 82.85) (width 0.25) (layer F.Cu) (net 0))
 (segment (start 57.85 81.95) (end 69.15 81.95) (width 0.25) (layer F.Cu) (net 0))
 (segment (start 69.15 82.85) (end 57.85 82.85) (width 0.25) (layer F.Cu) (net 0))
 (segment (start 70.85 81.95) (end 82.15 81.95) (width 0.25) (layer F.Cu) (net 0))
 (segment (start 71.5 82.85) (end 82.15 82.85) (width 0.25) (layer F.Cu) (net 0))
 (segment (start 70.85 82.85) (end 71.5 82.85) (width 0.25) (layer F.Cu) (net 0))
 (segment (start 83.85 81.95) (end 95.15 81.95) (width 0.25) (layer F.Cu) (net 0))
 (segment (start 84.5 82.85) (end 95.15 82.85) (width 0.25) (layer F.Cu) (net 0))
 (segment (start 83.85 82.85) (end 84.5 82.85) (width 0.25) (layer F.Cu) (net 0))
 (segment (start 97.5 81.95) (end 108.15 81.95) (width 0.25) (layer F.Cu) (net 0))
 (segment (start 96.85 81.95) (end 97.5 81.95) (width 0.25) (layer F.Cu) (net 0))
 (segment (start 108.15 82.85) (end 96.85 82.85) (width 0.25) (layer F.Cu) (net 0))
 (segment (start 109.85 81.95) (end 121.125 81.95) (width 0.25) (layer F.Cu) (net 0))
 (segment (start 121.125 82.85) (end 110 82.85) (width 0.25) (layer F.Cu) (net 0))
 (segment (start 110 82.85) (end 109.85 82.85) (width 0.25) (layer F.Cu) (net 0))
 (segment (start 122.825 81.95) (end 134.15 81.95) (width 0.25) (layer F.Cu) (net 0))
 (segment (start 123.225 82.85) (end 122.825 82.85) (width 0.25) (layer F.Cu) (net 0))
 (segment (start 134.15 82.85) (end 123.225 82.85) (width 0.25) (layer F.Cu) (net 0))
 (segment (start 135.85 81.95) (end 147.15 81.95) (width 0.25) (layer F.Cu) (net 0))
 (segment (start 147.15 82.85) (end 135.85 82.85) (width 0.25) (layer F.Cu) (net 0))
 (segment (start 148.85 81.95) (end 160.125 81.95) (width 0.25) (layer F.Cu) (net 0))
 (segment (start 160.125 82.85) (end 148.85 82.85) (width 0.25) (layer F.Cu) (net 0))
 (segment (start 161.825 81.95) (end 173.15 81.95) (width 0.25) (layer F.Cu) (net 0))
 (segment (start 173.15 82.85) (end 161.825 82.85) (width 0.25) (layer F.Cu) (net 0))
 (segment (start 174.85 81.95) (end 186.15 81.95) (width 0.25) (layer F.Cu) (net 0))
 (segment (start 186.15 82.85) (end 174.85 82.85) (width 0.25) (layer F.Cu) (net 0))
 (segment (start 188.5 81.95) (end 199.125 81.95) (width 0.25) (layer F.Cu) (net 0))
 (segment (start 187.85 81.95) (end 188.5 81.95) (width 0.25) (layer F.Cu) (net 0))
 (segment (start 199.125 82.85) (end 187.85 82.85) (width 0.25) (layer F.Cu) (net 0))
 (segment (start 200.825 81.95) (end 212.15 81.95) (width 0.25) (layer F.Cu) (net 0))
 (segment (start 212.15 82.85) (end 200.825 82.85) (width 0.25) (layer F.Cu) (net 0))
 (segment (start 213.85 81.95) (end 225.15 81.95) (width 0.25) (layer F.Cu) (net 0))
 (segment (start 225.15 82.85) (end 213.85 82.85) (width 0.25) (layer F.Cu) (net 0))
 (segment (start 226.85 81.95) (end 238.15 81.95) (width 0.25) (layer F.Cu) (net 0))
 (segment (start 238.15 82.85) (end 226.85 82.85) (width 0.25) (layer F.Cu) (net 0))
 (segment (start 240.5 81.95) (end 251.15 81.95) (width 0.25) (layer F.Cu) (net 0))
 (segment (start 239.85 81.95) (end 240.5 81.95) (width 0.25) (layer F.Cu) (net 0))
 (segment (start 251.15 82.85) (end 239.85 82.85) (width 0.25) (layer F.Cu) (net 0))
 (segment (start 252.85 81.95) (end 264.15 81.95) (width 0.25) (layer F.Cu) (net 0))
 (segment (start 264.15 82.85) (end 252.85 82.85) (width 0.25) (layer F.Cu) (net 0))
 (segment (start 265.85 81.95) (end 277.15 81.95) (width 0.25) (layer F.Cu) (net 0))
 (segment (start 276.5 82.85) (end 265.85 82.85) (width 0.25) (layer F.Cu) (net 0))
 (segment (start 277.15 82.85) (end 276.5 82.85) (width 0.25) (layer F.Cu) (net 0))
 (segment (start 278.85 81.95) (end 290.15 81.95) (width 0.25) (layer F.Cu) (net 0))
 (segment (start 290.15 82.85) (end 278.85 82.85) (width 0.25) (layer F.Cu) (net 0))
 (segment (start 291.85 81.95) (end 292.825 81.95) (width 0.25) (layer F.Cu) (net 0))
 (segment (start 293.275 81.5) (end 295 81.5) (width 0.25) (layer F.Cu) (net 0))
 (segment (start 292.825 81.95) (end 293.275 81.5) (width 0.25) (layer F.Cu) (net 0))
 (segment (start 291.85 82.85) (end 292.975 82.85) (width 0.25) (layer F.Cu) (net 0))
 (segment (start 292.975 82.85) (end 293.325 82.5) (width 0.25) (layer F.Cu) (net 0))
 (segment (start 295 81.5) (end 298.45 81.5) (width 0.25) (layer F.Cu) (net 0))
 (segment (start 294.7 82.5) (end 298.45 82.5) (width 0.25) (layer F.Cu) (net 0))
 (segment (start 294.7 82.5) (end 295 82.5) (width 0.25) (layer F.Cu) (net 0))
 (segment (start 293.325 82.5) (end 294.7 82.5) (width 0.25) (layer F.Cu) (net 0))
 (segment (start 295 83.5) (end 298.45 83.5) (width 0.5) (layer F.Cu) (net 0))
 (segment (start 295 84.5) (end 298.45 84.5) (width 0.5) (layer F.Cu) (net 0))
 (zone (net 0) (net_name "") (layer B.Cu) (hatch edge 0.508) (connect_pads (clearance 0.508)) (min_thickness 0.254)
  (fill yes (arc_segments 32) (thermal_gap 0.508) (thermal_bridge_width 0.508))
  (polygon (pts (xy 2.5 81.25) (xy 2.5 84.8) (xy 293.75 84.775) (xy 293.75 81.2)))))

